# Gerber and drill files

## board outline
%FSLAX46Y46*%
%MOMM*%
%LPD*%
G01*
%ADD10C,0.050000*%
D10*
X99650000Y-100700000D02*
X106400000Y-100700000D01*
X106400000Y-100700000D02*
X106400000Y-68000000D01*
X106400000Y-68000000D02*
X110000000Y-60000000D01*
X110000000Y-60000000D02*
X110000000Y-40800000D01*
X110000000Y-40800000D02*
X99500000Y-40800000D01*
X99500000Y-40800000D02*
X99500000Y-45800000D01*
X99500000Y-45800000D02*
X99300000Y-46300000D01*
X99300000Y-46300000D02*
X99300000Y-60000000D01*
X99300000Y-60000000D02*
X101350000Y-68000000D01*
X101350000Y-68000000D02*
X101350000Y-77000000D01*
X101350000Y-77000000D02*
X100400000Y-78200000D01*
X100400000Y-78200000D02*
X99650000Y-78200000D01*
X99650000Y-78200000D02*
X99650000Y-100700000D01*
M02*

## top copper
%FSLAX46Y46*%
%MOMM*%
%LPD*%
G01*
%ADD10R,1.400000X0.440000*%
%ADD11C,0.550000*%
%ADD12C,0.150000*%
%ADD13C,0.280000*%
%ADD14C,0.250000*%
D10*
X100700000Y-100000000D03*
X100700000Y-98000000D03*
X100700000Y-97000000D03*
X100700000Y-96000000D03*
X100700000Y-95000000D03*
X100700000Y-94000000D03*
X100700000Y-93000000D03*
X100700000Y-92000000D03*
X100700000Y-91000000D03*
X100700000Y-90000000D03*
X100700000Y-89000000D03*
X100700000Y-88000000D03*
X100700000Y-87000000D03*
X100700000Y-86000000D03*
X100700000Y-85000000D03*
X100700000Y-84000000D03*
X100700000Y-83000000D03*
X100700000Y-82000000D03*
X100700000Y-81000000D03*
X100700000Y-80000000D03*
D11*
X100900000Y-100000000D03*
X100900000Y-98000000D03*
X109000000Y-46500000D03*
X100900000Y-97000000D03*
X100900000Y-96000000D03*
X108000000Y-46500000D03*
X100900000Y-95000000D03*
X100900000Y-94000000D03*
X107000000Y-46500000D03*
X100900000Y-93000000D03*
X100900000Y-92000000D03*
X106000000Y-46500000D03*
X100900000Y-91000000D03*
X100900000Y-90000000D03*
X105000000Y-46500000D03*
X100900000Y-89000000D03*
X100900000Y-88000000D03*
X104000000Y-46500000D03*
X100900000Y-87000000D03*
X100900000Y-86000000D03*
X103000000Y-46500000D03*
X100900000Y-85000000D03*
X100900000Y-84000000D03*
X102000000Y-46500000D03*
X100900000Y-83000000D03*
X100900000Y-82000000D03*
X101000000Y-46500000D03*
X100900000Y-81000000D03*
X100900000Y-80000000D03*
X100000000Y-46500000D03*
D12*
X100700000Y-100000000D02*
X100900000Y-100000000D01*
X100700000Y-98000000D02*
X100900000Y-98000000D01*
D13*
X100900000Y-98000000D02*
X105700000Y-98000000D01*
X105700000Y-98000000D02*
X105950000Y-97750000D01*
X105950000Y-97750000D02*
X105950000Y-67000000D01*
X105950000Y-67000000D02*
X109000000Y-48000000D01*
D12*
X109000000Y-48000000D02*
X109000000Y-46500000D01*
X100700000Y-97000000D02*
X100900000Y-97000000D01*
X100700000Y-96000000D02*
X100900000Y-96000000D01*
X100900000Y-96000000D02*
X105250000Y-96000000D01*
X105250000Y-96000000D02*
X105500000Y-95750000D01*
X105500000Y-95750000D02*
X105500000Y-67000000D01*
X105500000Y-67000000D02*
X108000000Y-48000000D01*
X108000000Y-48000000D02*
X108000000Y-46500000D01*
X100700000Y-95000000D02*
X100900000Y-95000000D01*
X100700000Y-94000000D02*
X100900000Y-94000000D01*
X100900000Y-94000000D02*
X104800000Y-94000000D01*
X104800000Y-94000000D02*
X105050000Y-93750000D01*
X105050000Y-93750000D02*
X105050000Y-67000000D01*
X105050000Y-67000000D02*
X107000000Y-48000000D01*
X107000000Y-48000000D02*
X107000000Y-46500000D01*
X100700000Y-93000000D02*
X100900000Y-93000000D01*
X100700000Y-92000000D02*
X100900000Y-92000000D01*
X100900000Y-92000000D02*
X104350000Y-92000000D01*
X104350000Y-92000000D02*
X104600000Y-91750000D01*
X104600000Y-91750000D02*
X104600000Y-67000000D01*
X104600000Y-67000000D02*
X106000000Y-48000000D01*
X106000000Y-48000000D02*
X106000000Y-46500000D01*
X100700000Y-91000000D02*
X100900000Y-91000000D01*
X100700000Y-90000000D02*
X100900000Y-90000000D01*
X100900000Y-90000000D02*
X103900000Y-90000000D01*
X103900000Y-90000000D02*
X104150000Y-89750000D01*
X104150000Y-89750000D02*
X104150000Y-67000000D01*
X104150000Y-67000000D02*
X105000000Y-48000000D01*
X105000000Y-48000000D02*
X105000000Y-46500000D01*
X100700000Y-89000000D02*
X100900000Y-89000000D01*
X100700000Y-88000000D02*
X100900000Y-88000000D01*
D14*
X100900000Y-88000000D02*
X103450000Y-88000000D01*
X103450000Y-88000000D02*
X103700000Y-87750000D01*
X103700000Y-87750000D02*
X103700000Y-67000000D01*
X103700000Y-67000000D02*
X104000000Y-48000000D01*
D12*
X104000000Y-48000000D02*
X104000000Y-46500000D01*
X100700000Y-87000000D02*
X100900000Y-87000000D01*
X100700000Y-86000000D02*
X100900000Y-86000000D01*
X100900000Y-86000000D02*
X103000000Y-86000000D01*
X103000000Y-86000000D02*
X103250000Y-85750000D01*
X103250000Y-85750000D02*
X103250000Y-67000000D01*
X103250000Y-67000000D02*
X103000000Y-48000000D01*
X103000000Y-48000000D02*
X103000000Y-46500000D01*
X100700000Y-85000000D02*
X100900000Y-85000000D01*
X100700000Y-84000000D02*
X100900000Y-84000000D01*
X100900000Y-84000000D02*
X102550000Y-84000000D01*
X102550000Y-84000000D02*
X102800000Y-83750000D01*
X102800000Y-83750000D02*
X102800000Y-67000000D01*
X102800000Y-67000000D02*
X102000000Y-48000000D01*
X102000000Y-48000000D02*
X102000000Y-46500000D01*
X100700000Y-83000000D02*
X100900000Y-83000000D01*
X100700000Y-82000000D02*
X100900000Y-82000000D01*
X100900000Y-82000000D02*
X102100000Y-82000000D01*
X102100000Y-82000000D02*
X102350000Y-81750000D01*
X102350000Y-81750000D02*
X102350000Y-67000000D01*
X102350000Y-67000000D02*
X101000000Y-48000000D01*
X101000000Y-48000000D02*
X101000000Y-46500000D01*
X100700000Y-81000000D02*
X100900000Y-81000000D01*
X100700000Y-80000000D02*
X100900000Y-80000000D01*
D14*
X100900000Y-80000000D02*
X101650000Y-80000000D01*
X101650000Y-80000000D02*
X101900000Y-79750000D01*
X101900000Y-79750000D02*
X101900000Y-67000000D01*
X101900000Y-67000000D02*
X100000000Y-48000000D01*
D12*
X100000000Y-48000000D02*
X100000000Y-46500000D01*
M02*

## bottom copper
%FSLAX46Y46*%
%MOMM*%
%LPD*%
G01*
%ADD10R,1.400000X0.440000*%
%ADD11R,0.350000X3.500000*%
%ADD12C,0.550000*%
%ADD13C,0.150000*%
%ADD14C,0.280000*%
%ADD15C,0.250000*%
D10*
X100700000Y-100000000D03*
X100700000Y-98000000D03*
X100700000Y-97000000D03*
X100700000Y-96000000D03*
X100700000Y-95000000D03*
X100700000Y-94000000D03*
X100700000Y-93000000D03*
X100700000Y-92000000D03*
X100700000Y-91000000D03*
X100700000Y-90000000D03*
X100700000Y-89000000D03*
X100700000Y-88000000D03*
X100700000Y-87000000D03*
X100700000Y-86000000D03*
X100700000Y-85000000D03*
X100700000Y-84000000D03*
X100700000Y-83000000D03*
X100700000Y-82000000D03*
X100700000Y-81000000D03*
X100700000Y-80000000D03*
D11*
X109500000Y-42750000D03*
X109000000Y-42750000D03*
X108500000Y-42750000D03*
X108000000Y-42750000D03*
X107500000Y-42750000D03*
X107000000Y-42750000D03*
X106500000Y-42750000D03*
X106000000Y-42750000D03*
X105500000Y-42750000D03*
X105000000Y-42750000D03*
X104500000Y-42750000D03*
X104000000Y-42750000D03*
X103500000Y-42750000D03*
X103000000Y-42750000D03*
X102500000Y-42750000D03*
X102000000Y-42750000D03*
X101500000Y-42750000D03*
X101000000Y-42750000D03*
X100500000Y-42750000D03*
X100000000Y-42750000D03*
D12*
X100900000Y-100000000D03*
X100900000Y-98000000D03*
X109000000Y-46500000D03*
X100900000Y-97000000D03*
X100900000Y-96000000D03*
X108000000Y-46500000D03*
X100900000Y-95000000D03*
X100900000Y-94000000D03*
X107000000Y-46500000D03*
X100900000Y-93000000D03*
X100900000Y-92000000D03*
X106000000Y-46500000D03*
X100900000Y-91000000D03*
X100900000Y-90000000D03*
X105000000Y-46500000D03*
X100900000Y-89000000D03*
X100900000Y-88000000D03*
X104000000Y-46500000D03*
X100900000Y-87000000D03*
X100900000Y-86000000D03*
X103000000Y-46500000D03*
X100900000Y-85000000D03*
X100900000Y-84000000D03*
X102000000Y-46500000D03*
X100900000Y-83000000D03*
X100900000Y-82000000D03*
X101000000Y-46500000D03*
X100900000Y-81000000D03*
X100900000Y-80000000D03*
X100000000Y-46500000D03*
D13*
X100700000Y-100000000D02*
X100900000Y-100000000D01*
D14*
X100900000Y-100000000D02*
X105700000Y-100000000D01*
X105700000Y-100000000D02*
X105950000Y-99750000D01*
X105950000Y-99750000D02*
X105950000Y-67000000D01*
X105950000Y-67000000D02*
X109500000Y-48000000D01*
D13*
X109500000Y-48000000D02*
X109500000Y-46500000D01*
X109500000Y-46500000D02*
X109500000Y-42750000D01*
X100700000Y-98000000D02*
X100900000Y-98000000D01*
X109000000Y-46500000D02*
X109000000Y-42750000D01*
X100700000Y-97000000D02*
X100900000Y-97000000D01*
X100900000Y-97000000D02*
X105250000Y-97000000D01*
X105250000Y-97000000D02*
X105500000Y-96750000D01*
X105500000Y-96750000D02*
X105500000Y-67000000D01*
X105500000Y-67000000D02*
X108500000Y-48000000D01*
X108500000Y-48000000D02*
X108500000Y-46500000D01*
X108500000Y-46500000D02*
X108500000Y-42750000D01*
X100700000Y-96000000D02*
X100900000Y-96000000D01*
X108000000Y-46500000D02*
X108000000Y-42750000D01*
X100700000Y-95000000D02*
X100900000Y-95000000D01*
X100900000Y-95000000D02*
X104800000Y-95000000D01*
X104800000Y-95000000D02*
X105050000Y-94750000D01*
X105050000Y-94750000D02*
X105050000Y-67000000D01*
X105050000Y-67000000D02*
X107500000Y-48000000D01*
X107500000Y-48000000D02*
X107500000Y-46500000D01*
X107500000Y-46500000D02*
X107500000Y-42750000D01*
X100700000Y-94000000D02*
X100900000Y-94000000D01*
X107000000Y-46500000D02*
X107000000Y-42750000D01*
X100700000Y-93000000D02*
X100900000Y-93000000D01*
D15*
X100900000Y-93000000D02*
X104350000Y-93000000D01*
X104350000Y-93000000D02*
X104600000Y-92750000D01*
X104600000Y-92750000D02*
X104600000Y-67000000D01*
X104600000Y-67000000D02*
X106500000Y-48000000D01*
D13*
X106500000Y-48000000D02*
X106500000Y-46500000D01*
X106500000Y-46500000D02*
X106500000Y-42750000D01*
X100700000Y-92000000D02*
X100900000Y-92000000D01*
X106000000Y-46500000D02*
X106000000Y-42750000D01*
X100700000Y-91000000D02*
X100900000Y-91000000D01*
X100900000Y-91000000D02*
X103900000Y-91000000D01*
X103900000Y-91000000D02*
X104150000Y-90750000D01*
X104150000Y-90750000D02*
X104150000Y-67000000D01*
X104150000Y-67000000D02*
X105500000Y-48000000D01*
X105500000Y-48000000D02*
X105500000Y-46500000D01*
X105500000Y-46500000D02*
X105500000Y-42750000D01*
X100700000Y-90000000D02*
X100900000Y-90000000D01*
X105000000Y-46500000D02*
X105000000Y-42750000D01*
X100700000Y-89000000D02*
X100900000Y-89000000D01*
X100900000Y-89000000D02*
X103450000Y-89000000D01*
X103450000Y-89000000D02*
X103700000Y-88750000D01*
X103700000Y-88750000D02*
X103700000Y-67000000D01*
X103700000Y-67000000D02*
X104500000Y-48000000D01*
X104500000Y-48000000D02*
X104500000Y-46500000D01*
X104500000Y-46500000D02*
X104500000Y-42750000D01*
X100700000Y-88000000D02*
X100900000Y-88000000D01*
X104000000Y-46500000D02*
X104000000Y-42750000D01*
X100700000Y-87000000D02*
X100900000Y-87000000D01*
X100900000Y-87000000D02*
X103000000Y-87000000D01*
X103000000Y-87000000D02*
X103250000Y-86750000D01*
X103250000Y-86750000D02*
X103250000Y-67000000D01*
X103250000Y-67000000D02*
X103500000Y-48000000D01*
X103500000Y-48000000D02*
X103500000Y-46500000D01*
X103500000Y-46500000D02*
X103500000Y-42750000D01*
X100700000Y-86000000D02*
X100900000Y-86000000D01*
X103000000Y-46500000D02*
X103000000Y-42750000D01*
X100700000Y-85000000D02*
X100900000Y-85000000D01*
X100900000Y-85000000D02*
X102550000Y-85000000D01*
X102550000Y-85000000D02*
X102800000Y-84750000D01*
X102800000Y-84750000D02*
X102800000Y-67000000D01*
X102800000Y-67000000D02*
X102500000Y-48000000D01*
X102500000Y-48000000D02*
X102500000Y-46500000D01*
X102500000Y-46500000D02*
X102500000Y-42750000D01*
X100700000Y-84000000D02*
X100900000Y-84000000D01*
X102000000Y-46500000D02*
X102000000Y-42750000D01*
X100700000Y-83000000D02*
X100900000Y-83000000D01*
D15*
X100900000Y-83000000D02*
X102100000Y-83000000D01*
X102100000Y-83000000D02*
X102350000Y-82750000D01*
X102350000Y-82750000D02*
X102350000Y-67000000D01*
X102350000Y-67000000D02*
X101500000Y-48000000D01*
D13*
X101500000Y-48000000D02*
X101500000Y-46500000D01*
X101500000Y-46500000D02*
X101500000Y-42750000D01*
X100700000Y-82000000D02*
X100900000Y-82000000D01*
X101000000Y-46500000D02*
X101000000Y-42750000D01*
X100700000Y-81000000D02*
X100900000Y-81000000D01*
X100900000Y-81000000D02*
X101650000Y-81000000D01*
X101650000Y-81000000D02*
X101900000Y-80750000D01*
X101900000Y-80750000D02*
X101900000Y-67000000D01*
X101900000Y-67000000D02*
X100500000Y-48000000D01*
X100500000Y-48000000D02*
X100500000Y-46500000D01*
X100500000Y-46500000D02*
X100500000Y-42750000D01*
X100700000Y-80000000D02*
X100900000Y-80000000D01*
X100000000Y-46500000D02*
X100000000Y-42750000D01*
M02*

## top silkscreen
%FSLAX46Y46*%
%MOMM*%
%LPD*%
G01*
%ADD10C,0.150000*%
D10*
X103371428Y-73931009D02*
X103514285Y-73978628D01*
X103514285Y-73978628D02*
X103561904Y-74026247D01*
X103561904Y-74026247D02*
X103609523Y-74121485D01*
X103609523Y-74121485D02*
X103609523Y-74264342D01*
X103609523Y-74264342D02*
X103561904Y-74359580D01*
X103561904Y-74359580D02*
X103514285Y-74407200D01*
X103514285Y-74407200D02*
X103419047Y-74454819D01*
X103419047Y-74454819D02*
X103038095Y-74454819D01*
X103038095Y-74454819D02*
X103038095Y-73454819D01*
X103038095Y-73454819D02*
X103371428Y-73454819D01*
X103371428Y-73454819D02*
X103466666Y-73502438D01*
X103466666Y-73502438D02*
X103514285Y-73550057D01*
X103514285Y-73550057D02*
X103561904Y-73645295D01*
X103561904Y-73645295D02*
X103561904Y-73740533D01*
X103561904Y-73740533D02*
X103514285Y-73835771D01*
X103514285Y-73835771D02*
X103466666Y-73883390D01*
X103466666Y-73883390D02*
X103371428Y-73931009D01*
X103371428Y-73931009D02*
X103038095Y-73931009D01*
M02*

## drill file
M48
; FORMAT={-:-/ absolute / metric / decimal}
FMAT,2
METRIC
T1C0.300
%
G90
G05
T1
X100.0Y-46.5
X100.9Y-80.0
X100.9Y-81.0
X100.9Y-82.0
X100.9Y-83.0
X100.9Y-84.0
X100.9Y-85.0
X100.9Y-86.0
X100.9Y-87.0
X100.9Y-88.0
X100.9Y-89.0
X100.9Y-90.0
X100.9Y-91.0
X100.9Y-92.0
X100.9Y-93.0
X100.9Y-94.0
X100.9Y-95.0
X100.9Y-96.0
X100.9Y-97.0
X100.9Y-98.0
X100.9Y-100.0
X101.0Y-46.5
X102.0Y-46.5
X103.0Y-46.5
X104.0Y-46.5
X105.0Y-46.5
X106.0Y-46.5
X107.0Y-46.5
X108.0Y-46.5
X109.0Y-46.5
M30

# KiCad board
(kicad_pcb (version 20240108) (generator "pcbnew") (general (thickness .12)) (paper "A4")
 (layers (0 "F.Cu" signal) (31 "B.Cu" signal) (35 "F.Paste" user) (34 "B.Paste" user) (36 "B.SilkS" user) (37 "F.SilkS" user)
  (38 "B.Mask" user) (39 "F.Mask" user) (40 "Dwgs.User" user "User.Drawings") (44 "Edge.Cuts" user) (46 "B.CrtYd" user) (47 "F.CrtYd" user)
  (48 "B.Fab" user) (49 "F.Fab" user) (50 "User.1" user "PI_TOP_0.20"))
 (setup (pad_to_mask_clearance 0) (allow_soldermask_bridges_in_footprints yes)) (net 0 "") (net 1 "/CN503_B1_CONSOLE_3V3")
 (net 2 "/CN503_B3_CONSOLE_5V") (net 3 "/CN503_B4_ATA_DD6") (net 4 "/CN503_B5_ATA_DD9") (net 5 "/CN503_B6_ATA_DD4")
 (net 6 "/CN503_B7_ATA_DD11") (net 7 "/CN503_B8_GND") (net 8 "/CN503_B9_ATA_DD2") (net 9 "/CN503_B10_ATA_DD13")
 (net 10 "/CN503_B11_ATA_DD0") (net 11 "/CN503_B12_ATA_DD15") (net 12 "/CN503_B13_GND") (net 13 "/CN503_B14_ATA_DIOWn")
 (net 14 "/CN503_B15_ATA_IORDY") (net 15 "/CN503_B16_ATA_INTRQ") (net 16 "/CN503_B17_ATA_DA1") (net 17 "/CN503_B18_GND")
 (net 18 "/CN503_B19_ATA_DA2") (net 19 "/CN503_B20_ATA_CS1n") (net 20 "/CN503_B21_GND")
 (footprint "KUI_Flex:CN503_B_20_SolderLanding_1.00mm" (layer "F.Cu") (at 100.0 100.0)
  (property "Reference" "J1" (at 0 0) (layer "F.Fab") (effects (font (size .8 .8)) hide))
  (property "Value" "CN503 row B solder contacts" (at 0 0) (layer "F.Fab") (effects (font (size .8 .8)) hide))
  (pad "1" smd rect (at 0.7 0) (size 1.4 .44) (layers "F.Cu" "F.Mask") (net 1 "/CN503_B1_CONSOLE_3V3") (solder_mask_margin .29))
  (pad "1" smd rect (at 0.7 0) (size 1.4 .44) (layers "B.Cu" "B.Mask") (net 1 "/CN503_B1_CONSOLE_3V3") (solder_mask_margin .29))
  (pad "3" smd rect (at 0.7 -2) (size 1.4 .44) (layers "F.Cu" "F.Mask") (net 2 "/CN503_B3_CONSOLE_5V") (solder_mask_margin .29))
  (pad "3" smd rect (at 0.7 -2) (size 1.4 .44) (layers "B.Cu" "B.Mask") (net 2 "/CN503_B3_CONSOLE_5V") (solder_mask_margin .29))
  (pad "4" smd rect (at 0.7 -3) (size 1.4 .44) (layers "F.Cu" "F.Mask") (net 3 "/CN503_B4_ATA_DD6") (solder_mask_margin .29))
  (pad "4" smd rect (at 0.7 -3) (size 1.4 .44) (layers "B.Cu" "B.Mask") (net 3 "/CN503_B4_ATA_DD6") (solder_mask_margin .29))
  (pad "5" smd rect (at 0.7 -4) (size 1.4 .44) (layers "F.Cu" "F.Mask") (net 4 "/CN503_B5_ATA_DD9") (solder_mask_margin .29))
  (pad "5" smd rect (at 0.7 -4) (size 1.4 .44) (layers "B.Cu" "B.Mask") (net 4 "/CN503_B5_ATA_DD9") (solder_mask_margin .29))
  (pad "6" smd rect (at 0.7 -5) (size 1.4 .44) (layers "F.Cu" "F.Mask") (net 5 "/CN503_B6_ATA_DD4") (solder_mask_margin .29))
  (pad "6" smd rect (at 0.7 -5) (size 1.4 .44) (layers "B.Cu" "B.Mask") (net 5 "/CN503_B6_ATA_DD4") (solder_mask_margin .29))
  (pad "7" smd rect (at 0.7 -6) (size 1.4 .44) (layers "F.Cu" "F.Mask") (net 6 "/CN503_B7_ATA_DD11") (solder_mask_margin .29))
  (pad "7" smd rect (at 0.7 -6) (size 1.4 .44) (layers "B.Cu" "B.Mask") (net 6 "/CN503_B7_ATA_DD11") (solder_mask_margin .29))
  (pad "8" smd rect (at 0.7 -7) (size 1.4 .44) (layers "F.Cu" "F.Mask") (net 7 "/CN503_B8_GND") (solder_mask_margin .29))
  (pad "8" smd rect (at 0.7 -7) (size 1.4 .44) (layers "B.Cu" "B.Mask") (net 7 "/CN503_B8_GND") (solder_mask_margin .29))
  (pad "9" smd rect (at 0.7 -8) (size 1.4 .44) (layers "F.Cu" "F.Mask") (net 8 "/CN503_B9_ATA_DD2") (solder_mask_margin .29))
  (pad "9" smd rect (at 0.7 -8) (size 1.4 .44) (layers "B.Cu" "B.Mask") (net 8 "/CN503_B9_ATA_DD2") (solder_mask_margin .29))
  (pad "10" smd rect (at 0.7 -9) (size 1.4 .44) (layers "F.Cu" "F.Mask") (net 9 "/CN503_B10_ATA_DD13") (solder_mask_margin .29))
  (pad "10" smd rect (at 0.7 -9) (size 1.4 .44) (layers "B.Cu" "B.Mask") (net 9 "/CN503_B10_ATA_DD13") (solder_mask_margin .29))
  (pad "11" smd rect (at 0.7 -10) (size 1.4 .44) (layers "F.Cu" "F.Mask") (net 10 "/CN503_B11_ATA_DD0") (solder_mask_margin .29))
  (pad "11" smd rect (at 0.7 -10) (size 1.4 .44) (layers "B.Cu" "B.Mask") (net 10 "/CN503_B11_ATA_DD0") (solder_mask_margin .29))
  (pad "12" smd rect (at 0.7 -11) (size 1.4 .44) (layers "F.Cu" "F.Mask") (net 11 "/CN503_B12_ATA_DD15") (solder_mask_margin .29))
  (pad "12" smd rect (at 0.7 -11) (size 1.4 .44) (layers "B.Cu" "B.Mask") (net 11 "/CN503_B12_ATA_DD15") (solder_mask_margin .29))
  (pad "13" smd rect (at 0.7 -12) (size 1.4 .44) (layers "F.Cu" "F.Mask") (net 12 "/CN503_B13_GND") (solder_mask_margin .29))
  (pad "13" smd rect (at 0.7 -12) (size 1.4 .44) (layers "B.Cu" "B.Mask") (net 12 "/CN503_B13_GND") (solder_mask_margin .29))
  (pad "14" smd rect (at 0.7 -13) (size 1.4 .44) (layers "F.Cu" "F.Mask") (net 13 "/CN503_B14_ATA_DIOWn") (solder_mask_margin .29))
  (pad "14" smd rect (at 0.7 -13) (size 1.4 .44) (layers "B.Cu" "B.Mask") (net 13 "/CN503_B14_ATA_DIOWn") (solder_mask_margin .29))
  (pad "15" smd rect (at 0.7 -14) (size 1.4 .44) (layers "F.Cu" "F.Mask") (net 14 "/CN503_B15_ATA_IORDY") (solder_mask_margin .29))
  (pad "15" smd rect (at 0.7 -14) (size 1.4 .44) (layers "B.Cu" "B.Mask") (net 14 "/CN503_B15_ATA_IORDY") (solder_mask_margin .29))
  (pad "16" smd rect (at 0.7 -15) (size 1.4 .44) (layers "F.Cu" "F.Mask") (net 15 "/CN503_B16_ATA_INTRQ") (solder_mask_margin .29))
  (pad "16" smd rect (at 0.7 -15) (size 1.4 .44) (layers "B.Cu" "B.Mask") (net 15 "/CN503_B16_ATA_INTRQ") (solder_mask_margin .29))
  (pad "17" smd rect (at 0.7 -16) (size 1.4 .44) (layers "F.Cu" "F.Mask") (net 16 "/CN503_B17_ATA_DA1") (solder_mask_margin .29))
  (pad "17" smd rect (at 0.7 -16) (size 1.4 .44) (layers "B.Cu" "B.Mask") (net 16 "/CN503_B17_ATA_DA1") (solder_mask_margin .29))
  (pad "18" smd rect (at 0.7 -17) (size 1.4 .44) (layers "F.Cu" "F.Mask") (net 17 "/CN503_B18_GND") (solder_mask_margin .29))
  (pad "18" smd rect (at 0.7 -17) (size 1.4 .44) (layers "B.Cu" "B.Mask") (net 17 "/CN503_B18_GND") (solder_mask_margin .29))
  (pad "19" smd rect (at 0.7 -18) (size 1.4 .44) (layers "F.Cu" "F.Mask") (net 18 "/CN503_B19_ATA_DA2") (solder_mask_margin .29))
  (pad "19" smd rect (at 0.7 -18) (size 1.4 .44) (layers "B.Cu" "B.Mask") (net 18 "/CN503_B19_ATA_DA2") (solder_mask_margin .29))
  (pad "20" smd rect (at 0.7 -19) (size 1.4 .44) (layers "F.Cu" "F.Mask") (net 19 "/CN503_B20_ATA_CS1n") (solder_mask_margin .29))
  (pad "20" smd rect (at 0.7 -19) (size 1.4 .44) (layers "B.Cu" "B.Mask") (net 19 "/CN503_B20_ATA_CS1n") (solder_mask_margin .29))
  (pad "21" smd rect (at 0.7 -20) (size 1.4 .44) (layers "F.Cu" "F.Mask") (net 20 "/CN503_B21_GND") (solder_mask_margin .29))
  (pad "21" smd rect (at 0.7 -20) (size 1.4 .44) (layers "B.Cu" "B.Mask") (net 20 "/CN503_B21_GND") (solder_mask_margin .29)))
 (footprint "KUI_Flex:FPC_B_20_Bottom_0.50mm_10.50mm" (layer "F.Cu") (at 100.0 100.0)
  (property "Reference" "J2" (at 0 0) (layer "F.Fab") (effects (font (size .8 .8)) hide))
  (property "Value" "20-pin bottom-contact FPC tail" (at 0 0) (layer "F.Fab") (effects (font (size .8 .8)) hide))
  (pad "20" smd rect (at 9.5 -57.25) (size .35 3.5) (layers "B.Cu" "B.Mask") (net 1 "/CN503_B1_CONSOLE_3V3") (solder_mask_margin .10))
  (pad "19" smd rect (at 9 -57.25) (size .35 3.5) (layers "B.Cu" "B.Mask") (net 2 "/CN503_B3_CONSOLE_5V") (solder_mask_margin .10))
  (pad "18" smd rect (at 8.5 -57.25) (size .35 3.5) (layers "B.Cu" "B.Mask") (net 3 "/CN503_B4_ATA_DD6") (solder_mask_margin .10))
  (pad "17" smd rect (at 8 -57.25) (size .35 3.5) (layers "B.Cu" "B.Mask") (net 4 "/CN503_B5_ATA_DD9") (solder_mask_margin .10))
  (pad "16" smd rect (at 7.5 -57.25) (size .35 3.5) (layers "B.Cu" "B.Mask") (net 5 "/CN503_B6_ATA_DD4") (solder_mask_margin .10))
  (pad "15" smd rect (at 7 -57.25) (size .35 3.5) (layers "B.Cu" "B.Mask") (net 6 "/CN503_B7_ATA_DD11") (solder_mask_margin .10))
  (pad "14" smd rect (at 6.5 -57.25) (size .35 3.5) (layers "B.Cu" "B.Mask") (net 7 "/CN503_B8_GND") (solder_mask_margin .10))
  (pad "13" smd rect (at 6 -57.25) (size .35 3.5) (layers "B.Cu" "B.Mask") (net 8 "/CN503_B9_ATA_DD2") (solder_mask_margin .10))
  (pad "12" smd rect (at 5.5 -57.25) (size .35 3.5) (layers "B.Cu" "B.Mask") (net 9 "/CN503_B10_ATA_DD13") (solder_mask_margin .10))
  (pad "11" smd rect (at 5 -57.25) (size .35 3.5) (layers "B.Cu" "B.Mask") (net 10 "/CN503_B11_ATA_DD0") (solder_mask_margin .10))
  (pad "10" smd rect (at 4.5 -57.25) (size .35 3.5) (layers "B.Cu" "B.Mask") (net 11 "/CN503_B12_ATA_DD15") (solder_mask_margin .10))
  (pad "9" smd rect (at 4 -57.25) (size .35 3.5) (layers "B.Cu" "B.Mask") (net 12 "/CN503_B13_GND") (solder_mask_margin .10))
  (pad "8" smd rect (at 3.5 -57.25) (size .35 3.5) (layers "B.Cu" "B.Mask") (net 13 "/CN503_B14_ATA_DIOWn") (solder_mask_margin .10))
  (pad "7" smd rect (at 3 -57.25) (size .35 3.5) (layers "B.Cu" "B.Mask") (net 14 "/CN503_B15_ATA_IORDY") (solder_mask_margin .10))
  (pad "6" smd rect (at 2.5 -57.25) (size .35 3.5) (layers "B.Cu" "B.Mask") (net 15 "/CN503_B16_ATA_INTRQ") (solder_mask_margin .10))
  (pad "5" smd rect (at 2 -57.25) (size .35 3.5) (layers "B.Cu" "B.Mask") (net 16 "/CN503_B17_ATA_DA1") (solder_mask_margin .10))
  (pad "4" smd rect (at 1.5 -57.25) (size .35 3.5) (layers "B.Cu" "B.Mask") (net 17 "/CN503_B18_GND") (solder_mask_margin .10))
  (pad "3" smd rect (at 1 -57.25) (size .35 3.5) (layers "B.Cu" "B.Mask") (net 18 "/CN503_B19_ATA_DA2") (solder_mask_margin .10))
  (pad "2" smd rect (at 0.5 -57.25) (size .35 3.5) (layers "B.Cu" "B.Mask") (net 19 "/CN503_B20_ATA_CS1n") (solder_mask_margin .10))
  (pad "1" smd rect (at 0 -57.25) (size .35 3.5) (layers "B.Cu" "B.Mask") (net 20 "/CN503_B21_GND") (solder_mask_margin .10)))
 (segment (start 100.7 100) (end 100.9 100) (width 0.15) (layer "F.Cu") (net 1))
 (segment (start 100.7 100) (end 100.9 100) (width 0.15) (layer "B.Cu") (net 1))
 (segment (start 100.9 100) (end 105.7 100) (width 0.28) (layer "B.Cu") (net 1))
 (segment (start 105.7 100) (end 105.95 99.75) (width 0.28) (layer "B.Cu") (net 1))
 (segment (start 105.95 99.75) (end 105.95 67) (width 0.28) (layer "B.Cu") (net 1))
 (segment (start 105.95 67) (end 109.5 48) (width 0.28) (layer "B.Cu") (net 1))
 (segment (start 109.5 48) (end 109.5 46.5) (width 0.15) (layer "B.Cu") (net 1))
 (segment (start 109.5 46.5) (end 109.5 42.75) (width 0.15) (layer "B.Cu") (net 1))
 (segment (start 100.7 98) (end 100.9 98) (width 0.15) (layer "F.Cu") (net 2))
 (segment (start 100.7 98) (end 100.9 98) (width 0.15) (layer "B.Cu") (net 2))
 (segment (start 100.9 98) (end 105.7 98) (width 0.28) (layer "F.Cu") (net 2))
 (segment (start 105.7 98) (end 105.95 97.75) (width 0.28) (layer "F.Cu") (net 2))
 (segment (start 105.95 97.75) (end 105.95 67) (width 0.28) (layer "F.Cu") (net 2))
 (segment (start 105.95 67) (end 109 48) (width 0.28) (layer "F.Cu") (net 2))
 (segment (start 109 48) (end 109 46.5) (width 0.15) (layer "F.Cu") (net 2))
 (segment (start 109 46.5) (end 109 42.75) (width 0.15) (layer "B.Cu") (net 2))
 (segment (start 100.7 97) (end 100.9 97) (width 0.15) (layer "F.Cu") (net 3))
 (segment (start 100.7 97) (end 100.9 97) (width 0.15) (layer "B.Cu") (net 3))
 (segment (start 100.9 97) (end 105.25 97) (width 0.15) (layer "B.Cu") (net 3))
 (segment (start 105.25 97) (end 105.5 96.75) (width 0.15) (layer "B.Cu") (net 3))
 (segment (start 105.5 96.75) (end 105.5 67) (width 0.15) (layer "B.Cu") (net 3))
 (segment (start 105.5 67) (end 108.5 48) (width 0.15) (layer "B.Cu") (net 3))
 (segment (start 108.5 48) (end 108.5 46.5) (width 0.15) (layer "B.Cu") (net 3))
 (segment (start 108.5 46.5) (end 108.5 42.75) (width 0.15) (layer "B.Cu") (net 3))
 (segment (start 100.7 96) (end 100.9 96) (width 0.15) (layer "F.Cu") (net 4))
 (segment (start 100.7 96) (end 100.9 96) (width 0.15) (layer "B.Cu") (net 4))
 (segment (start 100.9 96) (end 105.25 96) (width 0.15) (layer "F.Cu") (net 4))
 (segment (start 105.25 96) (end 105.5 95.75) (width 0.15) (layer "F.Cu") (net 4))
 (segment (start 105.5 95.75) (end 105.5 67) (width 0.15) (layer "F.Cu") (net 4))
 (segment (start 105.5 67) (end 108 48) (width 0.15) (layer "F.Cu") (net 4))
 (segment (start 108 48) (end 108 46.5) (width 0.15) (layer "F.Cu") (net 4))
 (segment (start 108 46.5) (end 108 42.75) (width 0.15) (layer "B.Cu") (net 4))
 (segment (start 100.7 95) (end 100.9 95) (width 0.15) (layer "F.Cu") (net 5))
 (segment (start 100.7 95) (end 100.9 95) (width 0.15) (layer "B.Cu") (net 5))
 (segment (start 100.9 95) (end 104.8 95) (width 0.15) (layer "B.Cu") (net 5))
 (segment (start 104.8 95) (end 105.05 94.75) (width 0.15) (layer "B.Cu") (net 5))
 (segment (start 105.05 94.75) (end 105.05 67) (width 0.15) (layer "B.Cu") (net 5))
 (segment (start 105.05 67) (end 107.5 48) (width 0.15) (layer "B.Cu") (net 5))
 (segment (start 107.5 48) (end 107.5 46.5) (width 0.15) (layer "B.Cu") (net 5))
 (segment (start 107.5 46.5) (end 107.5 42.75) (width 0.15) (layer "B.Cu") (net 5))
 (segment (start 100.7 94) (end 100.9 94) (width 0.15) (layer "F.Cu") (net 6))
 (segment (start 100.7 94) (end 100.9 94) (width 0.15) (layer "B.Cu") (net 6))
 (segment (start 100.9 94) (end 104.8 94) (width 0.15) (layer "F.Cu") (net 6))
 (segment (start 104.8 94) (end 105.05 93.75) (width 0.15) (layer "F.Cu") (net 6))
 (segment (start 105.05 93.75) (end 105.05 67) (width 0.15) (layer "F.Cu") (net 6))
 (segment (start 105.05 67) (end 107 48) (width 0.15) (layer "F.Cu") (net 6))
 (segment (start 107 48) (end 107 46.5) (width 0.15) (layer "F.Cu") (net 6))
 (segment (start 107 46.5) (end 107 42.75) (width 0.15) (layer "B.Cu") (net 6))
 (segment (start 100.7 93) (end 100.9 93) (width 0.15) (layer "F.Cu") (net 7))
 (segment (start 100.7 93) (end 100.9 93) (width 0.15) (layer "B.Cu") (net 7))
 (segment (start 100.9 93) (end 104.35 93) (width 0.25) (layer "B.Cu") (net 7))
 (segment (start 104.35 93) (end 104.6 92.75) (width 0.25) (layer "B.Cu") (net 7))
 (segment (start 104.6 92.75) (end 104.6 67) (width 0.25) (layer "B.Cu") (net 7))
 (segment (start 104.6 67) (end 106.5 48) (width 0.25) (layer "B.Cu") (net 7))
 (segment (start 106.5 48) (end 106.5 46.5) (width 0.15) (layer "B.Cu") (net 7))
 (segment (start 106.5 46.5) (end 106.5 42.75) (width 0.15) (layer "B.Cu") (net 7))
 (segment (start 100.7 92) (end 100.9 92) (width 0.15) (layer "F.Cu") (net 8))
 (segment (start 100.7 92) (end 100.9 92) (width 0.15) (layer "B.Cu") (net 8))
 (segment (start 100.9 92) (end 104.35 92) (width 0.15) (layer "F.Cu") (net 8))
 (segment (start 104.35 92) (end 104.6 91.75) (width 0.15) (layer "F.Cu") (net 8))
 (segment (start 104.6 91.75) (end 104.6 67) (width 0.15) (layer "F.Cu") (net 8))
 (segment (start 104.6 67) (end 106 48) (width 0.15) (layer "F.Cu") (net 8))
 (segment (start 106 48) (end 106 46.5) (width 0.15) (layer "F.Cu") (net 8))
 (segment (start 106 46.5) (end 106 42.75) (width 0.15) (layer "B.Cu") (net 8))
 (segment (start 100.7 91) (end 100.9 91) (width 0.15) (layer "F.Cu") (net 9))
 (segment (start 100.7 91) (end 100.9 91) (width 0.15) (layer "B.Cu") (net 9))
 (segment (start 100.9 91) (end 103.9 91) (width 0.15) (layer "B.Cu") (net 9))
 (segment (start 103.9 91) (end 104.15 90.75) (width 0.15) (layer "B.Cu") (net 9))
 (segment (start 104.15 90.75) (end 104.15 67) (width 0.15) (layer "B.Cu") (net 9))
 (segment (start 104.15 67) (end 105.5 48) (width 0.15) (layer "B.Cu") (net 9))
 (segment (start 105.5 48) (end 105.5 46.5) (width 0.15) (layer "B.Cu") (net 9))
 (segment (start 105.5 46.5) (end 105.5 42.75) (width 0.15) (layer "B.Cu") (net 9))
 (segment (start 100.7 90) (end 100.9 90) (width 0.15) (layer "F.Cu") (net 10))
 (segment (start 100.7 90) (end 100.9 90) (width 0.15) (layer "B.Cu") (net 10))
 (segment (start 100.9 90) (end 103.9 90) (width 0.15) (layer "F.Cu") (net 10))
 (segment (start 103.9 90) (end 104.15 89.75) (width 0.15) (layer "F.Cu") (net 10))
 (segment (start 104.15 89.75) (end 104.15 67) (width 0.15) (layer "F.Cu") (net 10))
 (segment (start 104.15 67) (end 105 48) (width 0.15) (layer "F.Cu") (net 10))
 (segment (start 105 48) (end 105 46.5) (width 0.15) (layer "F.Cu") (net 10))
 (segment (start 105 46.5) (end 105 42.75) (width 0.15) (layer "B.Cu") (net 10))
 (segment (start 100.7 89) (end 100.9 89) (width 0.15) (layer "F.Cu") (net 11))
 (segment (start 100.7 89) (end 100.9 89) (width 0.15) (layer "B.Cu") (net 11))
 (segment (start 100.9 89) (end 103.45 89) (width 0.15) (layer "B.Cu") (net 11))
 (segment (start 103.45 89) (end 103.7 88.75) (width 0.15) (layer "B.Cu") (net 11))
 (segment (start 103.7 88.75) (end 103.7 67) (width 0.15) (layer "B.Cu") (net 11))
 (segment (start 103.7 67) (end 104.5 48) (width 0.15) (layer "B.Cu") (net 11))
 (segment (start 104.5 48) (end 104.5 46.5) (width 0.15) (layer "B.Cu") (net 11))
 (segment (start 104.5 46.5) (end 104.5 42.75) (width 0.15) (layer "B.Cu") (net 11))
 (segment (start 100.7 88) (end 100.9 88) (width 0.15) (layer "F.Cu") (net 12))
 (segment (start 100.7 88) (end 100.9 88) (width 0.15) (layer "B.Cu") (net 12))
 (segment (start 100.9 88) (end 103.45 88) (width 0.25) (layer "F.Cu") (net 12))
 (segment (start 103.45 88) (end 103.7 87.75) (width 0.25) (layer "F.Cu") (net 12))
 (segment (start 103.7 87.75) (end 103.7 67) (width 0.25) (layer "F.Cu") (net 12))
 (segment (start 103.7 67) (end 104 48) (width 0.25) (layer "F.Cu") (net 12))
 (segment (start 104 48) (end 104 46.5) (width 0.15) (layer "F.Cu") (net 12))
 (segment (start 104 46.5) (end 104 42.75) (width 0.15) (layer "B.Cu") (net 12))
 (segment (start 100.7 87) (end 100.9 87) (width 0.15) (layer "F.Cu") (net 13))
 (segment (start 100.7 87) (end 100.9 87) (width 0.15) (layer "B.Cu") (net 13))
 (segment (start 100.9 87) (end 103 87) (width 0.15) (layer "B.Cu") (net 13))
 (segment (start 103 87) (end 103.25 86.75) (width 0.15) (layer "B.Cu") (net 13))
 (segment (start 103.25 86.75) (end 103.25 67) (width 0.15) (layer "B.Cu") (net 13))
 (segment (start 103.25 67) (end 103.5 48) (width 0.15) (layer "B.Cu") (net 13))
 (segment (start 103.5 48) (end 103.5 46.5) (width 0.15) (layer "B.Cu") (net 13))
 (segment (start 103.5 46.5) (end 103.5 42.75) (width 0.15) (layer "B.Cu") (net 13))
 (segment (start 100.7 86) (end 100.9 86) (width 0.15) (layer "F.Cu") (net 14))
 (segment (start 100.7 86) (end 100.9 86) (width 0.15) (layer "B.Cu") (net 14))
 (segment (start 100.9 86) (end 103 86) (width 0.15) (layer "F.Cu") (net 14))
 (segment (start 103 86) (end 103.25 85.75) (width 0.15) (layer "F.Cu") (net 14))
 (segment (start 103.25 85.75) (end 103.25 67) (width 0.15) (layer "F.Cu") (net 14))
 (segment (start 103.25 67) (end 103 48) (width 0.15) (layer "F.Cu") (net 14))
 (segment (start 103 48) (end 103 46.5) (width 0.15) (layer "F.Cu") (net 14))
 (segment (start 103 46.5) (end 103 42.75) (width 0.15) (layer "B.Cu") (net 14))
 (segment (start 100.7 85) (end 100.9 85) (width 0.15) (layer "F.Cu") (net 15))
 (segment (start 100.7 85) (end 100.9 85) (width 0.15) (layer "B.Cu") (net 15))
 (segment (start 100.9 85) (end 102.55 85) (width 0.15) (layer "B.Cu") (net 15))
 (segment (start 102.55 85) (end 102.8 84.75) (width 0.15) (layer "B.Cu") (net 15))
 (segment (start 102.8 84.75) (end 102.8 67) (width 0.15) (layer "B.Cu") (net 15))
 (segment (start 102.8 67) (end 102.5 48) (width 0.15) (layer "B.Cu") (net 15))
 (segment (start 102.5 48) (end 102.5 46.5) (width 0.15) (layer "B.Cu") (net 15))
 (segment (start 102.5 46.5) (end 102.5 42.75) (width 0.15) (layer "B.Cu") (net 15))
 (segment (start 100.7 84) (end 100.9 84) (width 0.15) (layer "F.Cu") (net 16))
 (segment (start 100.7 84) (end 100.9 84) (width 0.15) (layer "B.Cu") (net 16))
 (segment (start 100.9 84) (end 102.55 84) (width 0.15) (layer "F.Cu") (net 16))
 (segment (start 102.55 84) (end 102.8 83.75) (width 0.15) (layer "F.Cu") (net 16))
 (segment (start 102.8 83.75) (end 102.8 67) (width 0.15) (layer "F.Cu") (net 16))
 (segment (start 102.8 67) (end 102 48) (width 0.15) (layer "F.Cu") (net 16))
 (segment (start 102 48) (end 102 46.5) (width 0.15) (layer "F.Cu") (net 16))
 (segment (start 102 46.5) (end 102 42.75) (width 0.15) (layer "B.Cu") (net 16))
 (segment (start 100.7 83) (end 100.9 83) (width 0.15) (layer "F.Cu") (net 17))
 (segment (start 100.7 83) (end 100.9 83) (width 0.15) (layer "B.Cu") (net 17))
 (segment (start 100.9 83) (end 102.1 83) (width 0.25) (layer "B.Cu") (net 17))
 (segment (start 102.1 83) (end 102.35 82.75) (width 0.25) (layer "B.Cu") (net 17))
 (segment (start 102.35 82.75) (end 102.35 67) (width 0.25) (layer "B.Cu") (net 17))
 (segment (start 102.35 67) (end 101.5 48) (width 0.25) (layer "B.Cu") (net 17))
 (segment (start 101.5 48) (end 101.5 46.5) (width 0.15) (layer "B.Cu") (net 17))
 (segment (start 101.5 46.5) (end 101.5 42.75) (width 0.15) (layer "B.Cu") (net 17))
 (segment (start 100.7 82) (end 100.9 82) (width 0.15) (layer "F.Cu") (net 18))
 (segment (start 100.7 82) (end 100.9 82) (width 0.15) (layer "B.Cu") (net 18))
 (segment (start 100.9 82) (end 102.1 82) (width 0.15) (layer "F.Cu") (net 18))
 (segment (start 102.1 82) (end 102.35 81.75) (width 0.15) (layer "F.Cu") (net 18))
 (segment (start 102.35 81.75) (end 102.35 67) (width 0.15) (layer "F.Cu") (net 18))
 (segment (start 102.35 67) (end 101 48) (width 0.15) (layer "F.Cu") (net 18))
 (segment (start 101 48) (end 101 46.5) (width 0.15) (layer "F.Cu") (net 18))
 (segment (start 101 46.5) (end 101 42.75) (width 0.15) (layer "B.Cu") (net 18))
 (segment (start 100.7 81) (end 100.9 81) (width 0.15) (layer "F.Cu") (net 19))
 (segment (start 100.7 81) (end 100.9 81) (width 0.15) (layer "B.Cu") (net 19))
 (segment (start 100.9 81) (end 101.65 81) (width 0.15) (layer "B.Cu") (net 19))
 (segment (start 101.65 81) (end 101.9 80.75) (width 0.15) (layer "B.Cu") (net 19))
 (segment (start 101.9 80.75) (end 101.9 67) (width 0.15) (layer "B.Cu") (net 19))
 (segment (start 101.9 67) (end 100.5 48) (width 0.15) (layer "B.Cu") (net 19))
 (segment (start 100.5 48) (end 100.5 46.5) (width 0.15) (layer "B.Cu") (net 19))
 (segment (start 100.5 46.5) (end 100.5 42.75) (width 0.15) (layer "B.Cu") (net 19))
 (segment (start 100.7 80) (end 100.9 80) (width 0.15) (layer "F.Cu") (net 20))
 (segment (start 100.7 80) (end 100.9 80) (width 0.15) (layer "B.Cu") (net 20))
 (segment (start 100.9 80) (end 101.65 80) (width 0.25) (layer "F.Cu") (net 20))
 (segment (start 101.65 80) (end 101.9 79.75) (width 0.25) (layer "F.Cu") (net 20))
 (segment (start 101.9 79.75) (end 101.9 67) (width 0.25) (layer "F.Cu") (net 20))
 (segment (start 101.9 67) (end 100 48) (width 0.25) (layer "F.Cu") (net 20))
 (segment (start 100 48) (end 100 46.5) (width 0.15) (layer "F.Cu") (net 20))
 (segment (start 100 46.5) (end 100 42.75) (width 0.15) (layer "B.Cu") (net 20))
 (via (at 100.9 100) (size .55) (drill .3) (layers "F.Cu" "B.Cu") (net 1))
 (via (at 100.9 98) (size .55) (drill .3) (layers "F.Cu" "B.Cu") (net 2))
 (via (at 109 46.5) (size .55) (drill .3) (layers "F.Cu" "B.Cu") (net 2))
 (via (at 100.9 97) (size .55) (drill .3) (layers "F.Cu" "B.Cu") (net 3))
 (via (at 100.9 96) (size .55) (drill .3) (layers "F.Cu" "B.Cu") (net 4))
 (via (at 108 46.5) (size .55) (drill .3) (layers "F.Cu" "B.Cu") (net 4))
 (via (at 100.9 95) (size .55) (drill .3) (layers "F.Cu" "B.Cu") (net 5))
 (via (at 100.9 94) (size .55) (drill .3) (layers "F.Cu" "B.Cu") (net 6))
 (via (at 107 46.5) (size .55) (drill .3) (layers "F.Cu" "B.Cu") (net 6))
 (via (at 100.9 93) (size .55) (drill .3) (layers "F.Cu" "B.Cu") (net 7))
 (via (at 100.9 92) (size .55) (drill .3) (layers "F.Cu" "B.Cu") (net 8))
 (via (at 106 46.5) (size .55) (drill .3) (layers "F.Cu" "B.Cu") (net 8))
 (via (at 100.9 91) (size .55) (drill .3) (layers "F.Cu" "B.Cu") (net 9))
 (via (at 100.9 90) (size .55) (drill .3) (layers "F.Cu" "B.Cu") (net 10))
 (via (at 105 46.5) (size .55) (drill .3) (layers "F.Cu" "B.Cu") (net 10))
 (via (at 100.9 89) (size .55) (drill .3) (layers "F.Cu" "B.Cu") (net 11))
 (via (at 100.9 88) (size .55) (drill .3) (layers "F.Cu" "B.Cu") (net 12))
 (via (at 104 46.5) (size .55) (drill .3) (layers "F.Cu" "B.Cu") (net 12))
 (via (at 100.9 87) (size .55) (drill .3) (layers "F.Cu" "B.Cu") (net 13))
 (via (at 100.9 86) (size .55) (drill .3) (layers "F.Cu" "B.Cu") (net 14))
 (via (at 103 46.5) (size .55) (drill .3) (layers "F.Cu" "B.Cu") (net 14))
 (via (at 100.9 85) (size .55) (drill .3) (layers "F.Cu" "B.Cu") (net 15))
 (via (at 100.9 84) (size .55) (drill .3) (layers "F.Cu" "B.Cu") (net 16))
 (via (at 102 46.5) (size .55) (drill .3) (layers "F.Cu" "B.Cu") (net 16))
 (via (at 100.9 83) (size .55) (drill .3) (layers "F.Cu" "B.Cu") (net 17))
 (via (at 100.9 82) (size .55) (drill .3) (layers "F.Cu" "B.Cu") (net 18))
 (via (at 101 46.5) (size .55) (drill .3) (layers "F.Cu" "B.Cu") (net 18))
 (via (at 100.9 81) (size .55) (drill .3) (layers "F.Cu" "B.Cu") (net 19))
 (via (at 100.9 80) (size .55) (drill .3) (layers "F.Cu" "B.Cu") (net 20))
 (via (at 100 46.5) (size .55) (drill .3) (layers "F.Cu" "B.Cu") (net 20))
 (gr_line (start 99.65 100.7) (end 106.4 100.7) (stroke (width .05) (type default)) (layer "Edge.Cuts"))
 (gr_line (start 106.4 100.7) (end 106.4 68) (stroke (width .05) (type default)) (layer "Edge.Cuts"))
 (gr_line (start 106.4 68) (end 110 60) (stroke (width .05) (type default)) (layer "Edge.Cuts"))
 (gr_line (start 110 60) (end 110 40.8) (stroke (width .05) (type default)) (layer "Edge.Cuts"))
 (gr_line (start 110 40.8) (end 99.5 40.8) (stroke (width .05) (type default)) (layer "Edge.Cuts"))
 (gr_line (start 99.5 40.8) (end 99.5 45.8) (stroke (width .05) (type default)) (layer "Edge.Cuts"))
 (gr_line (start 99.5 45.8) (end 99.3 46.3) (stroke (width .05) (type default)) (layer "Edge.Cuts"))
 (gr_line (start 99.3 46.3) (end 99.3 60) (stroke (width .05) (type default)) (layer "Edge.Cuts"))
 (gr_line (start 99.3 60) (end 101.35 68) (stroke (width .05) (type default)) (layer "Edge.Cuts"))
 (gr_line (start 101.35 68) (end 101.35 77) (stroke (width .05) (type default)) (layer "Edge.Cuts"))
 (gr_line (start 101.35 77) (end 100.4 78.2) (stroke (width .05) (type default)) (layer "Edge.Cuts"))
 (gr_line (start 100.4 78.2) (end 99.65 78.2) (stroke (width .05) (type default)) (layer "Edge.Cuts"))
 (gr_line (start 99.65 78.2) (end 99.65 100.7) (stroke (width .05) (type default)) (layer "Edge.Cuts"))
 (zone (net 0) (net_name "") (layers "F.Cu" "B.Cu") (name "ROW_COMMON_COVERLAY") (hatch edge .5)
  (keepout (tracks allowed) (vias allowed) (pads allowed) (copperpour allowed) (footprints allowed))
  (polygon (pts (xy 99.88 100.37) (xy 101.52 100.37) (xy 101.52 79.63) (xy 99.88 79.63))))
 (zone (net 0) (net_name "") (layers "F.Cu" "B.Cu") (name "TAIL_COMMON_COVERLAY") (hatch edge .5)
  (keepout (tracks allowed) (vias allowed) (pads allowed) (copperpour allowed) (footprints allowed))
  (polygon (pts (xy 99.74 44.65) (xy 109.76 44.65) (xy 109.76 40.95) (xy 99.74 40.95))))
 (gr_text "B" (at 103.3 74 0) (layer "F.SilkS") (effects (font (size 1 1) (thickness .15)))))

